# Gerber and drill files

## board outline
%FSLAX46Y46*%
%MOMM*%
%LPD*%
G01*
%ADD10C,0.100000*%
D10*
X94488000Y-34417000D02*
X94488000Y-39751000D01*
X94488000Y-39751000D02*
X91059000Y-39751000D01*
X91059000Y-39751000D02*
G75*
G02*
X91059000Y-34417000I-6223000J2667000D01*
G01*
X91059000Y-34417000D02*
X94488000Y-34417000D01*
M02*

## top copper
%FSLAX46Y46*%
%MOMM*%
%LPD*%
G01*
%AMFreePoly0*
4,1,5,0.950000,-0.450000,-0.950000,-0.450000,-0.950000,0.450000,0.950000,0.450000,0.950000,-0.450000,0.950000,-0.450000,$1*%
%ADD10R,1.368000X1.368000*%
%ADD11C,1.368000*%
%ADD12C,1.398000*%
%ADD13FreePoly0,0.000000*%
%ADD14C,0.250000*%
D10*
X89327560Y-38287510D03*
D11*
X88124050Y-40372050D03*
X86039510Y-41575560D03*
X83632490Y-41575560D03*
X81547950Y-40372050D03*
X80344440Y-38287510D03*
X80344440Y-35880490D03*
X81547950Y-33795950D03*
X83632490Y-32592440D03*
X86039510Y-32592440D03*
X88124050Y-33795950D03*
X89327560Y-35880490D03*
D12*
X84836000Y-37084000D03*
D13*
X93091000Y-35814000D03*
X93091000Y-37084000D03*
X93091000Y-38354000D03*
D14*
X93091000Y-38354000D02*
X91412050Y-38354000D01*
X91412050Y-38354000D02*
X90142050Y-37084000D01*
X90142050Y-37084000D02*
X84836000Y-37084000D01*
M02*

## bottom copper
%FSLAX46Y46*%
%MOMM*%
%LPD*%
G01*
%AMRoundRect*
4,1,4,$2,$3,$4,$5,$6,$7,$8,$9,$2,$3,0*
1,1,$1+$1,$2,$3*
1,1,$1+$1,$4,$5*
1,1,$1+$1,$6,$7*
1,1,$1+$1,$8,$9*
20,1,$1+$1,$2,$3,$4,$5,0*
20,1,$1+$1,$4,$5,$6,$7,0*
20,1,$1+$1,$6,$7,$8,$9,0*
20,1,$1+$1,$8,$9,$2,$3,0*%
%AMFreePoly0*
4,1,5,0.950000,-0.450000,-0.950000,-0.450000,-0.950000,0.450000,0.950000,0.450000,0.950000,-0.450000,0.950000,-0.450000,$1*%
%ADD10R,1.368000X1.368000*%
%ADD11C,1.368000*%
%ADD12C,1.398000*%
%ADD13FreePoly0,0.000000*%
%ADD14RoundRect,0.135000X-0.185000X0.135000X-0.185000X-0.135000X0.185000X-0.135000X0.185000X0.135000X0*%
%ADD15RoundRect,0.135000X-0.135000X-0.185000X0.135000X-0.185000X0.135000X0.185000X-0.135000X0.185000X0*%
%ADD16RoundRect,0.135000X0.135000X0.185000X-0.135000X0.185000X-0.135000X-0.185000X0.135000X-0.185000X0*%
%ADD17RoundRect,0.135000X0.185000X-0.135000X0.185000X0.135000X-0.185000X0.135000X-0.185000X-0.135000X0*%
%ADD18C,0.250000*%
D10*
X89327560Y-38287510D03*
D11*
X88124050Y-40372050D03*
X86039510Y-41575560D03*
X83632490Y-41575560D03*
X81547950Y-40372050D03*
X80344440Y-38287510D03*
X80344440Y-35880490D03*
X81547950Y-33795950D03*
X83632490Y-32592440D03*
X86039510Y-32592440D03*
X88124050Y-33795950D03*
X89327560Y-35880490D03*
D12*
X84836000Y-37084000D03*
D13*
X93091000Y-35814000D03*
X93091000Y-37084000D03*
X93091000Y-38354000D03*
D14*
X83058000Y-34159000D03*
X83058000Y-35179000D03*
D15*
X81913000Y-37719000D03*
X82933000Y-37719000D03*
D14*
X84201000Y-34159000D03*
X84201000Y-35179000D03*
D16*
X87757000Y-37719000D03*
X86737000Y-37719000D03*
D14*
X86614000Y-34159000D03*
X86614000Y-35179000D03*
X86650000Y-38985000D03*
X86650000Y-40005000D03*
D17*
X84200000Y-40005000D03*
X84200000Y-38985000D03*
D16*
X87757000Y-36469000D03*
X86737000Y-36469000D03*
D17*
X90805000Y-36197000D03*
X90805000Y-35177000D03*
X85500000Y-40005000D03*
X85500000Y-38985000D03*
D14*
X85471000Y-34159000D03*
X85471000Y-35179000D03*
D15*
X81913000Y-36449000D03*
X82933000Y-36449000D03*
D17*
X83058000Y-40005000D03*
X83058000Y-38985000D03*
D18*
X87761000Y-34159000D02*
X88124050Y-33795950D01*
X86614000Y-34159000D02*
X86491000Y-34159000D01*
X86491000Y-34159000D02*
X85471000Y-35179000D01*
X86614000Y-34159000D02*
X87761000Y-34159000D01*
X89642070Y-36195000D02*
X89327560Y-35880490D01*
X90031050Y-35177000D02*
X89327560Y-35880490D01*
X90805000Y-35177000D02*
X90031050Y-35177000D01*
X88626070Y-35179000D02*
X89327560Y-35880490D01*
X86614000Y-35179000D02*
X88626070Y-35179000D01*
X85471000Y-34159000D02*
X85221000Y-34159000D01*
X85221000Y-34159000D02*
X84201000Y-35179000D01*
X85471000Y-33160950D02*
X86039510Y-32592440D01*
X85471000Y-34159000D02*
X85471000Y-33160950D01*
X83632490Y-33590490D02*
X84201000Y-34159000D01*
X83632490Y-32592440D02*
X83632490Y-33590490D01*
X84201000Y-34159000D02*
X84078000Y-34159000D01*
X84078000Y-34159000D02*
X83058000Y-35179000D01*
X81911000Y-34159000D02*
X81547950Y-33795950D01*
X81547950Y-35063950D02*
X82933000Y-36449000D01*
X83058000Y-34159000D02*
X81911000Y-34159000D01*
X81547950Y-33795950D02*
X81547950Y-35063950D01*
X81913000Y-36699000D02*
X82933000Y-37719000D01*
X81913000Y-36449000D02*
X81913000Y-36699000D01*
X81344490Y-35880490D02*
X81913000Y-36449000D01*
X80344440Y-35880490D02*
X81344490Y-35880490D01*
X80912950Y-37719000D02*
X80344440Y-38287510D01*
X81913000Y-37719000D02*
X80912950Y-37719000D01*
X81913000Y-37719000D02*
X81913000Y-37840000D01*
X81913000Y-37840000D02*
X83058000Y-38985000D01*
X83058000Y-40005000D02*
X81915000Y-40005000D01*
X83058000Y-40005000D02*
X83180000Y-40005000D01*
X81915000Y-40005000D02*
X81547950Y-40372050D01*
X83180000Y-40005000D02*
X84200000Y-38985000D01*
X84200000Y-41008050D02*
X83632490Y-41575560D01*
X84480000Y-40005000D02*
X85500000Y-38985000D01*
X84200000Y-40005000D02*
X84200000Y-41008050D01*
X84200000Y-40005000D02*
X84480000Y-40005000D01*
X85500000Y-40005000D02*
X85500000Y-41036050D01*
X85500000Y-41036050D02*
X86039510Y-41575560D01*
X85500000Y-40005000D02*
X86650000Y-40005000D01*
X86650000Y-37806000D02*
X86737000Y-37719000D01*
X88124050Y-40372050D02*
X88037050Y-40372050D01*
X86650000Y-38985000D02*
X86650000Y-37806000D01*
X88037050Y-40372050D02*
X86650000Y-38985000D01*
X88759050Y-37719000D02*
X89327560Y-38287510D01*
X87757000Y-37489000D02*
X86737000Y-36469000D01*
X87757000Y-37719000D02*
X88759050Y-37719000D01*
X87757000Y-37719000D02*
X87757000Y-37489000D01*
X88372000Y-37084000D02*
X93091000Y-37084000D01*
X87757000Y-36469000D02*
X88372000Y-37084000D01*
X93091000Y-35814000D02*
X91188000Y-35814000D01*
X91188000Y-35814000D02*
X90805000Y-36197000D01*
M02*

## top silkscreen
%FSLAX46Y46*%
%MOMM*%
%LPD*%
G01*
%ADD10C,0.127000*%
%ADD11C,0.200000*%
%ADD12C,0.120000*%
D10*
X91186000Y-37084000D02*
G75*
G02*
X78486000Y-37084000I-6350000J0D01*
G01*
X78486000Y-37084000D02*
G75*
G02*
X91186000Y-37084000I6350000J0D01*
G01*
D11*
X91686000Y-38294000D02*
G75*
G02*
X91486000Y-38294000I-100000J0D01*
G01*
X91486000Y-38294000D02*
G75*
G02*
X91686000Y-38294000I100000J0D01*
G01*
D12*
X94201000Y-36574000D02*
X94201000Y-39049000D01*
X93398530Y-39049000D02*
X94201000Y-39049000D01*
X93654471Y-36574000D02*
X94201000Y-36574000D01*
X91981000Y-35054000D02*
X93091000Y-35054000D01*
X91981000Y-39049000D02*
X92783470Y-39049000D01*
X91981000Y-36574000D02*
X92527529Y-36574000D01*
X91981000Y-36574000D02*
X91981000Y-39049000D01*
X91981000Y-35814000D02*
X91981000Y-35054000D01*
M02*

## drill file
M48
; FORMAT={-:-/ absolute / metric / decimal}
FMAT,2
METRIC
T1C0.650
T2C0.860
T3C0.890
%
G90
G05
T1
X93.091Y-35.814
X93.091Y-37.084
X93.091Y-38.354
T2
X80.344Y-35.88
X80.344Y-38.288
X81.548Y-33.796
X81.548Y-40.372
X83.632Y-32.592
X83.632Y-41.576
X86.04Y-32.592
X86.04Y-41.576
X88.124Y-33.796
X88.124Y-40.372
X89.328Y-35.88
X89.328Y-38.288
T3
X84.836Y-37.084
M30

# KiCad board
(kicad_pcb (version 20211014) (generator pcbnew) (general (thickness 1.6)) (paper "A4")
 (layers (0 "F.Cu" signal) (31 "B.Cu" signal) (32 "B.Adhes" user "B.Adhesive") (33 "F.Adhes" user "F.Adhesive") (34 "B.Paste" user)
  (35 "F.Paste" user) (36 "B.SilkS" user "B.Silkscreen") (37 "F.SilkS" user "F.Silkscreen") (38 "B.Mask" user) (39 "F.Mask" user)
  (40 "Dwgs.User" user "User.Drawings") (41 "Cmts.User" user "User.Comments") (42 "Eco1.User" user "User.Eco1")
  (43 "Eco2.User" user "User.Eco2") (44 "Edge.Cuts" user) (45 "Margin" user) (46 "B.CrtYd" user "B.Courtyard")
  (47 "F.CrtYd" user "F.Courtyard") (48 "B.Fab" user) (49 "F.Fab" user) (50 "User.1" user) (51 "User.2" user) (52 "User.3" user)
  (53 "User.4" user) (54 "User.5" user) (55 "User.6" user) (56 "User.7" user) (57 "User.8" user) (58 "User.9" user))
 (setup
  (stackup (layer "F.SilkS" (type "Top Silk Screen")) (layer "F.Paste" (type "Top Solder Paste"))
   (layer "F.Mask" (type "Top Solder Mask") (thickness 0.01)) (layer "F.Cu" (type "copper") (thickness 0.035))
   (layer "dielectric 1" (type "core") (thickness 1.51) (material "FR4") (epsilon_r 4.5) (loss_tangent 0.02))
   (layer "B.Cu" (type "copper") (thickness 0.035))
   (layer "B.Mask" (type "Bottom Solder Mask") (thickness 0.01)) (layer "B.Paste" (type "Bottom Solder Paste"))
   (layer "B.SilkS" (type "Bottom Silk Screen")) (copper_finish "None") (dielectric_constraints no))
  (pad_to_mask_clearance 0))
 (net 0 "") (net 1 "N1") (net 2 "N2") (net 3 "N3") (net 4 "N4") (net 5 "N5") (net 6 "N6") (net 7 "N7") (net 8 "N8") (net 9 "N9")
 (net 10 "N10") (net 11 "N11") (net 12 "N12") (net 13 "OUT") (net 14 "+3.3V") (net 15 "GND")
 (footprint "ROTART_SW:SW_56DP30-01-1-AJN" (layer "F.Cu") (at 84.836 37.084)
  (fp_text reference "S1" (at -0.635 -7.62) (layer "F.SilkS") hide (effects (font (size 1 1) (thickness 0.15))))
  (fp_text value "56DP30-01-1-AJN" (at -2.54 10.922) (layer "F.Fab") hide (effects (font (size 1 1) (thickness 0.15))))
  (fp_circle (center 0 0) (end 6.35 0) (layer "F.SilkS") (width 0.127) (fill none))
  (fp_circle (center 6.75 1.21) (end 6.85 1.21) (layer "F.SilkS") (width 0.2) (fill none))
  (pad "1" thru_hole rect (at 4.49156 1.20351) (size 1.368 1.368) (drill 0.86) (layers *.Cu *.Mask) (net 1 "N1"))
  (pad "2" thru_hole circle (at 3.28805 3.28805) (size 1.368 1.368) (drill 0.86) (layers *.Cu *.Mask) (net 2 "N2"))
  (pad "3" thru_hole circle (at 1.20351 4.49156) (size 1.368 1.368) (drill 0.86) (layers *.Cu *.Mask) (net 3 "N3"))
  (pad "4" thru_hole circle (at -1.20351 4.49156) (size 1.368 1.368) (drill 0.86) (layers *.Cu *.Mask) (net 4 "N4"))
  (pad "5" thru_hole circle (at -3.28805 3.28805) (size 1.368 1.368) (drill 0.86) (layers *.Cu *.Mask) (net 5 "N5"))
  (pad "6" thru_hole circle (at -4.49156 1.20351) (size 1.368 1.368) (drill 0.86) (layers *.Cu *.Mask) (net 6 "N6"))
  (pad "7" thru_hole circle (at -4.49156 -1.20351) (size 1.368 1.368) (drill 0.86) (layers *.Cu *.Mask) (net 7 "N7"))
  (pad "8" thru_hole circle (at -3.28805 -3.28805) (size 1.368 1.368) (drill 0.86) (layers *.Cu *.Mask) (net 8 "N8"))
  (pad "9" thru_hole circle (at -1.20351 -4.49156) (size 1.368 1.368) (drill 0.86) (layers *.Cu *.Mask) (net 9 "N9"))
  (pad "10" thru_hole circle (at 1.20351 -4.49156) (size 1.368 1.368) (drill 0.86) (layers *.Cu *.Mask) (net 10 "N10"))
  (pad "11" thru_hole circle (at 3.28805 -3.28805) (size 1.368 1.368) (drill 0.86) (layers *.Cu *.Mask) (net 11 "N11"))
  (pad "12" thru_hole circle (at 4.49156 -1.20351) (size 1.368 1.368) (drill 0.86) (layers *.Cu *.Mask) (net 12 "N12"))
  (pad "C" thru_hole circle (at 0 0) (size 1.398 1.398) (drill 0.89) (layers *.Cu *.Mask) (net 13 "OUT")))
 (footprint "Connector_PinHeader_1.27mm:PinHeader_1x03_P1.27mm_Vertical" (layer "F.Cu") (at 93.091 35.814)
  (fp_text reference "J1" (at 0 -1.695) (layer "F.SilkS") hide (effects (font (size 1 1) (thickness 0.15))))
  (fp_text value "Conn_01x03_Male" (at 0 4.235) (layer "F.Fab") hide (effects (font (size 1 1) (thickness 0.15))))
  (fp_line (start 1.11 0.76) (end 1.11 3.235) (layer "F.SilkS") (width 0.12))
  (fp_line (start 0.30753 3.235) (end 1.11 3.235) (layer "F.SilkS") (width 0.12))
  (fp_line (start 0.563471 0.76) (end 1.11 0.76) (layer "F.SilkS") (width 0.12))
  (fp_line (start -1.11 -0.76) (end 0 -0.76) (layer "F.SilkS") (width 0.12))
  (fp_line (start -1.11 3.235) (end -0.30753 3.235) (layer "F.SilkS") (width 0.12))
  (fp_line (start -1.11 0.76) (end -0.563471 0.76) (layer "F.SilkS") (width 0.12))
  (fp_line (start -1.11 0.76) (end -1.11 3.235) (layer "F.SilkS") (width 0.12))
  (fp_line (start -1.11 0) (end -1.11 -0.76) (layer "F.SilkS") (width 0.12))
  (pad "1" thru_hole custom (at 0 0) (size 1.9 0.9) (drill 0.65) (layers *.Cu *.Mask) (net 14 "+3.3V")
   (options (clearance outline) (anchor rect)) (primitives))
  (pad "2" thru_hole custom (at 0 1.27) (size 1.9 0.9) (drill 0.65) (layers *.Cu *.Mask) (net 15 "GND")
   (options (clearance outline) (anchor rect)) (primitives))
  (pad "3" thru_hole custom (at 0 2.54) (size 1.9 0.9) (drill 0.65) (layers *.Cu *.Mask) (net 13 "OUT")
   (options (clearance outline) (anchor rect)) (primitives)))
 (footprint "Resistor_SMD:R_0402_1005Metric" (layer "B.Cu") (at 83.058 34.669 -90)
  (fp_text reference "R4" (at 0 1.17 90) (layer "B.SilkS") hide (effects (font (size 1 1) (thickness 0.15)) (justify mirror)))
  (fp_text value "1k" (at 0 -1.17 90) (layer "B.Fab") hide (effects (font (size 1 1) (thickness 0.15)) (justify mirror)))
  (pad "1" smd roundrect (at -0.51 0 270) (size 0.54 0.64) (layers "B.Cu" "B.Paste" "B.Mask") (roundrect_rratio 0.25) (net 8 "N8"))
  (pad "2" smd roundrect (at 0.51 0 270) (size 0.54 0.64) (layers "B.Cu" "B.Paste" "B.Mask") (roundrect_rratio 0.25) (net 9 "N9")))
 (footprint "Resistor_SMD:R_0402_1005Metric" (layer "B.Cu") (at 82.423 37.719)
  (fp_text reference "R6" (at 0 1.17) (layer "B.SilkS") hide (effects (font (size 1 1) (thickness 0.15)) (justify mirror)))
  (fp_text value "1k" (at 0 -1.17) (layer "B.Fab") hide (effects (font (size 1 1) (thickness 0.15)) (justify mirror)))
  (pad "1" smd roundrect (at -0.51 0) (size 0.54 0.64) (layers "B.Cu" "B.Paste" "B.Mask") (roundrect_rratio 0.25) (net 6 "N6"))
  (pad "2" smd roundrect (at 0.51 0) (size 0.54 0.64) (layers "B.Cu" "B.Paste" "B.Mask") (roundrect_rratio 0.25) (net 7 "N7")))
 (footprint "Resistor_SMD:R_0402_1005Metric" (layer "B.Cu") (at 84.201 34.669 -90)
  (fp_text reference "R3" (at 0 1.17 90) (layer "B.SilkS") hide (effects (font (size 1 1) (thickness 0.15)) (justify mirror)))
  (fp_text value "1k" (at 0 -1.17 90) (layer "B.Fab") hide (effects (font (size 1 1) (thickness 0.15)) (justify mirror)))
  (pad "1" smd roundrect (at -0.51 0 270) (size 0.54 0.64) (layers "B.Cu" "B.Paste" "B.Mask") (roundrect_rratio 0.25) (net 9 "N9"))
  (pad "2" smd roundrect (at 0.51 0 270) (size 0.54 0.64) (layers "B.Cu" "B.Paste" "B.Mask") (roundrect_rratio 0.25) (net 10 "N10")))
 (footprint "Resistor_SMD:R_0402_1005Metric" (layer "B.Cu") (at 87.247 37.719 180)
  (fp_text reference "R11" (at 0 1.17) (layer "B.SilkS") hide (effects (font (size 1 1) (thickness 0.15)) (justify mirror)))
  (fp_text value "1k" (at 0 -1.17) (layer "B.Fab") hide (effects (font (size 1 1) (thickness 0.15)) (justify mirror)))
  (pad "1" smd roundrect (at -0.51 0 180) (size 0.54 0.64) (layers "B.Cu" "B.Paste" "B.Mask") (roundrect_rratio 0.25) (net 1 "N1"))
  (pad "2" smd roundrect (at 0.51 0 180) (size 0.54 0.64) (layers "B.Cu" "B.Paste" "B.Mask") (roundrect_rratio 0.25) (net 2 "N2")))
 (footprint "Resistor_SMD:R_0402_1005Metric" (layer "B.Cu") (at 86.614 34.669 -90)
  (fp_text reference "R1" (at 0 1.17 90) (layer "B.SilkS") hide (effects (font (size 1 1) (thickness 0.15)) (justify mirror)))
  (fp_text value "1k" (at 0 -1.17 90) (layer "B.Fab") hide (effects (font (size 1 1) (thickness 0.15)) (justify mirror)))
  (pad "1" smd roundrect (at -0.51 0 270) (size 0.54 0.64) (layers "B.Cu" "B.Paste" "B.Mask") (roundrect_rratio 0.25) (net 11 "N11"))
  (pad "2" smd roundrect (at 0.51 0 270) (size 0.54 0.64) (layers "B.Cu" "B.Paste" "B.Mask") (roundrect_rratio 0.25) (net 12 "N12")))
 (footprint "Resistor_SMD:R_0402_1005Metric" (layer "B.Cu") (at 86.65 39.495 -90)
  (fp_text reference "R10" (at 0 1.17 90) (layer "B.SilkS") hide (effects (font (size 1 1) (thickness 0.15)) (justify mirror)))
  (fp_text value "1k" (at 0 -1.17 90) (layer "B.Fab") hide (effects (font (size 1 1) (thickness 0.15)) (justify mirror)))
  (pad "1" smd roundrect (at -0.51 0 270) (size 0.54 0.64) (layers "B.Cu" "B.Paste" "B.Mask") (roundrect_rratio 0.25) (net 2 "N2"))
  (pad "2" smd roundrect (at 0.51 0 270) (size 0.54 0.64) (layers "B.Cu" "B.Paste" "B.Mask") (roundrect_rratio 0.25) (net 3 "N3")))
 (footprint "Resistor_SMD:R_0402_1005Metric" (layer "B.Cu") (at 84.2 39.495 90)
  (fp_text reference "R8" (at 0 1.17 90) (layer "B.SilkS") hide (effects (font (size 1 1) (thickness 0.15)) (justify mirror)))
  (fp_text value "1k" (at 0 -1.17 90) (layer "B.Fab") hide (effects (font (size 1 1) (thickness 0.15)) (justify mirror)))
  (pad "1" smd roundrect (at -0.51 0 90) (size 0.54 0.64) (layers "B.Cu" "B.Paste" "B.Mask") (roundrect_rratio 0.25) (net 4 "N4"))
  (pad "2" smd roundrect (at 0.51 0 90) (size 0.54 0.64) (layers "B.Cu" "B.Paste" "B.Mask") (roundrect_rratio 0.25) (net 5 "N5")))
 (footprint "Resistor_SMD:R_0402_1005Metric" (layer "B.Cu") (at 87.247 36.469 180)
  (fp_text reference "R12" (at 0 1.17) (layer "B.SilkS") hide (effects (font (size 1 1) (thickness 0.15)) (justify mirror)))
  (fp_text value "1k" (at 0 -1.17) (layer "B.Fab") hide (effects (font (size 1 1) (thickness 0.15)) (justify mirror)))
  (pad "1" smd roundrect (at -0.51 0 180) (size 0.54 0.64) (layers "B.Cu" "B.Paste" "B.Mask") (roundrect_rratio 0.25) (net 15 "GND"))
  (pad "2" smd roundrect (at 0.51 0 180) (size 0.54 0.64) (layers "B.Cu" "B.Paste" "B.Mask") (roundrect_rratio 0.25) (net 1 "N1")))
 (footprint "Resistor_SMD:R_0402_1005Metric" (layer "B.Cu") (at 90.805 35.687 90)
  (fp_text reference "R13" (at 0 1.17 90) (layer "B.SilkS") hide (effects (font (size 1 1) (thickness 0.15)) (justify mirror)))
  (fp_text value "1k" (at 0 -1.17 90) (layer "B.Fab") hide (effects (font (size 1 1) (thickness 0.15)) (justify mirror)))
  (pad "1" smd roundrect (at -0.51 0 90) (size 0.54 0.64) (layers "B.Cu" "B.Paste" "B.Mask") (roundrect_rratio 0.25) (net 14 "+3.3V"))
  (pad "2" smd roundrect (at 0.51 0 90) (size 0.54 0.64) (layers "B.Cu" "B.Paste" "B.Mask") (roundrect_rratio 0.25) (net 12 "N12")))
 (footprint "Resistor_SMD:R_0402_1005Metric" (layer "B.Cu") (at 85.5 39.495 90)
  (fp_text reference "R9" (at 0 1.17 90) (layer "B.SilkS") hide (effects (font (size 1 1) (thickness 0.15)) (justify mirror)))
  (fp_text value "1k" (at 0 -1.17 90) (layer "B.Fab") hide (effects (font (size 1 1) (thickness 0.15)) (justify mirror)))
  (pad "1" smd roundrect (at -0.51 0 90) (size 0.54 0.64) (layers "B.Cu" "B.Paste" "B.Mask") (roundrect_rratio 0.25) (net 3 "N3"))
  (pad "2" smd roundrect (at 0.51 0 90) (size 0.54 0.64) (layers "B.Cu" "B.Paste" "B.Mask") (roundrect_rratio 0.25) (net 4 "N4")))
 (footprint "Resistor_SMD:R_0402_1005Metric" (layer "B.Cu") (at 85.471 34.669 -90)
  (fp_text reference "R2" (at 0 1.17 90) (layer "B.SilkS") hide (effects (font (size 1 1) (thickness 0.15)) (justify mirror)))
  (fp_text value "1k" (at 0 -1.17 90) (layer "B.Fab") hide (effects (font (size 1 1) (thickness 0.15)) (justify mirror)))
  (pad "1" smd roundrect (at -0.51 0 270) (size 0.54 0.64) (layers "B.Cu" "B.Paste" "B.Mask") (roundrect_rratio 0.25) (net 10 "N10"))
  (pad "2" smd roundrect (at 0.51 0 270) (size 0.54 0.64) (layers "B.Cu" "B.Paste" "B.Mask") (roundrect_rratio 0.25) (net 11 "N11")))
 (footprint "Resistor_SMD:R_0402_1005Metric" (layer "B.Cu") (at 82.423 36.449)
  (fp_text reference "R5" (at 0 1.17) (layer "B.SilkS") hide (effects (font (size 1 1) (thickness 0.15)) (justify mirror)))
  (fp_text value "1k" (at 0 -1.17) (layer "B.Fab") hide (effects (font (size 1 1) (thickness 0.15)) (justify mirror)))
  (pad "1" smd roundrect (at -0.51 0) (size 0.54 0.64) (layers "B.Cu" "B.Paste" "B.Mask") (roundrect_rratio 0.25) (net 7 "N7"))
  (pad "2" smd roundrect (at 0.51 0) (size 0.54 0.64) (layers "B.Cu" "B.Paste" "B.Mask") (roundrect_rratio 0.25) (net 8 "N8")))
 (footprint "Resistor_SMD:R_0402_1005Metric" (layer "B.Cu") (at 83.058 39.495 90)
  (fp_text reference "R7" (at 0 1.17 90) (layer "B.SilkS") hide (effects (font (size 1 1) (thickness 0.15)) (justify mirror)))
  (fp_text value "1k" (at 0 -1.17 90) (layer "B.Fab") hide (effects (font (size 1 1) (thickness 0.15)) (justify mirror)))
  (pad "1" smd roundrect (at -0.51 0 90) (size 0.54 0.64) (layers "B.Cu" "B.Paste" "B.Mask") (roundrect_rratio 0.25) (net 5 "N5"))
  (pad "2" smd roundrect (at 0.51 0 90) (size 0.54 0.64) (layers "B.Cu" "B.Paste" "B.Mask") (roundrect_rratio 0.25) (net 6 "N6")))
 (gr_line (start 94.488 34.417) (end 94.488 39.751) (layer "Edge.Cuts") (width 0.1))
 (gr_line (start 94.488 39.751) (end 91.059 39.751) (layer "Edge.Cuts") (width 0.1))
 (gr_arc (start 91.059 39.751) (mid 78.065578 37.084) (end 91.059 34.417) (layer "Edge.Cuts") (width 0.1))
 (gr_line (start 91.059 34.417) (end 94.488 34.417) (layer "Edge.Cuts") (width 0.1))
 (segment (start 93.091 38.354) (end 91.41205 38.354) (width 0.25) (layer "F.Cu") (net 13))
 (segment (start 91.41205 38.354) (end 90.14205 37.084) (width 0.25) (layer "F.Cu") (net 13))
 (segment (start 90.14205 37.084) (end 84.836 37.084) (width 0.25) (layer "F.Cu") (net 13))
 (segment (start 87.761 34.159) (end 88.12405 33.79595) (width 0.25) (layer "B.Cu") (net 11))
 (segment (start 86.614 34.159) (end 86.491 34.159) (width 0.25) (layer "B.Cu") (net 11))
 (segment (start 86.491 34.159) (end 85.471 35.179) (width 0.25) (layer "B.Cu") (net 11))
 (segment (start 86.614 34.159) (end 87.761 34.159) (width 0.25) (layer "B.Cu") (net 11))
 (segment (start 89.64207 36.195) (end 89.32756 35.88049) (width 0.25) (layer "B.Cu") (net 12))
 (segment (start 90.03105 35.177) (end 89.32756 35.88049) (width 0.25) (layer "B.Cu") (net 12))
 (segment (start 90.805 35.177) (end 90.03105 35.177) (width 0.25) (layer "B.Cu") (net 12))
 (segment (start 88.62607 35.179) (end 89.32756 35.88049) (width 0.25) (layer "B.Cu") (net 12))
 (segment (start 86.614 35.179) (end 88.62607 35.179) (width 0.25) (layer "B.Cu") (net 12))
 (segment (start 85.471 34.159) (end 85.221 34.159) (width 0.25) (layer "B.Cu") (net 10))
 (segment (start 85.221 34.159) (end 84.201 35.179) (width 0.25) (layer "B.Cu") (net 10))
 (segment (start 85.471 33.16095) (end 86.03951 32.59244) (width 0.25) (layer "B.Cu") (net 10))
 (segment (start 85.471 34.159) (end 85.471 33.16095) (width 0.25) (layer "B.Cu") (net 10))
 (segment (start 83.63249 33.59049) (end 84.201 34.159) (width 0.25) (layer "B.Cu") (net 9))
 (segment (start 83.63249 32.59244) (end 83.63249 33.59049) (width 0.25) (layer "B.Cu") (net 9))
 (segment (start 84.201 34.159) (end 84.078 34.159) (width 0.25) (layer "B.Cu") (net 9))
 (segment (start 84.078 34.159) (end 83.058 35.179) (width 0.25) (layer "B.Cu") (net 9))
 (segment (start 81.911 34.159) (end 81.54795 33.79595) (width 0.25) (layer "B.Cu") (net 8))
 (segment (start 81.54795 35.06395) (end 82.933 36.449) (width 0.25) (layer "B.Cu") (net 8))
 (segment (start 83.058 34.159) (end 81.911 34.159) (width 0.25) (layer "B.Cu") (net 8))
 (segment (start 81.54795 33.79595) (end 81.54795 35.06395) (width 0.25) (layer "B.Cu") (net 8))
 (segment (start 81.913 36.699) (end 82.933 37.719) (width 0.25) (layer "B.Cu") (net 7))
 (segment (start 81.913 36.449) (end 81.913 36.699) (width 0.25) (layer "B.Cu") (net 7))
 (segment (start 81.34449 35.88049) (end 81.913 36.449) (width 0.25) (layer "B.Cu") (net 7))
 (segment (start 80.34444 35.88049) (end 81.34449 35.88049) (width 0.25) (layer "B.Cu") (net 7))
 (segment (start 80.91295 37.719) (end 80.34444 38.28751) (width 0.25) (layer "B.Cu") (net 6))
 (segment (start 81.913 37.719) (end 80.91295 37.719) (width 0.25) (layer "B.Cu") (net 6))
 (segment (start 81.913 37.719) (end 81.913 37.84) (width 0.25) (layer "B.Cu") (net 6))
 (segment (start 81.913 37.84) (end 83.058 38.985) (width 0.25) (layer "B.Cu") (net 6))
 (segment (start 83.058 40.005) (end 81.915 40.005) (width 0.25) (layer "B.Cu") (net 5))
 (segment (start 83.058 40.005) (end 83.18 40.005) (width 0.25) (layer "B.Cu") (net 5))
 (segment (start 81.915 40.005) (end 81.54795 40.37205) (width 0.25) (layer "B.Cu") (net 5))
 (segment (start 83.18 40.005) (end 84.2 38.985) (width 0.25) (layer "B.Cu") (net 5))
 (segment (start 84.2 41.00805) (end 83.63249 41.57556) (width 0.25) (layer "B.Cu") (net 4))
 (segment (start 84.48 40.005) (end 85.5 38.985) (width 0.25) (layer "B.Cu") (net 4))
 (segment (start 84.2 40.005) (end 84.2 41.00805) (width 0.25) (layer "B.Cu") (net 4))
 (segment (start 84.2 40.005) (end 84.48 40.005) (width 0.25) (layer "B.Cu") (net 4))
 (segment (start 85.5 40.005) (end 85.5 41.03605) (width 0.25) (layer "B.Cu") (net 3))
 (segment (start 85.5 41.03605) (end 86.03951 41.57556) (width 0.25) (layer "B.Cu") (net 3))
 (segment (start 85.5 40.005) (end 86.65 40.005) (width 0.25) (layer "B.Cu") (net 3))
 (segment (start 86.65 37.806) (end 86.737 37.719) (width 0.25) (layer "B.Cu") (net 2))
 (segment (start 88.12405 40.37205) (end 88.03705 40.37205) (width 0.25) (layer "B.Cu") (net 2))
 (segment (start 86.65 38.985) (end 86.65 37.806) (width 0.25) (layer "B.Cu") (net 2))
 (segment (start 88.03705 40.37205) (end 86.65 38.985) (width 0.25) (layer "B.Cu") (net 2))
 (segment (start 88.75905 37.719) (end 89.32756 38.28751) (width 0.25) (layer "B.Cu") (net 1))
 (segment (start 87.757 37.489) (end 86.737 36.469) (width 0.25) (layer "B.Cu") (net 1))
 (segment (start 87.757 37.719) (end 88.75905 37.719) (width 0.25) (layer "B.Cu") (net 1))
 (segment (start 87.757 37.719) (end 87.757 37.489) (width 0.25) (layer "B.Cu") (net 1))
 (segment (start 88.372 37.084) (end 93.091 37.084) (width 0.25) (layer "B.Cu") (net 15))
 (segment (start 87.757 36.469) (end 88.372 37.084) (width 0.25) (layer "B.Cu") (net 15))
 (segment (start 93.091 35.814) (end 91.188 35.814) (width 0.25) (layer "B.Cu") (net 14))
 (segment (start 91.188 35.814) (end 90.805 36.197) (width 0.25) (layer "B.Cu") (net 14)))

